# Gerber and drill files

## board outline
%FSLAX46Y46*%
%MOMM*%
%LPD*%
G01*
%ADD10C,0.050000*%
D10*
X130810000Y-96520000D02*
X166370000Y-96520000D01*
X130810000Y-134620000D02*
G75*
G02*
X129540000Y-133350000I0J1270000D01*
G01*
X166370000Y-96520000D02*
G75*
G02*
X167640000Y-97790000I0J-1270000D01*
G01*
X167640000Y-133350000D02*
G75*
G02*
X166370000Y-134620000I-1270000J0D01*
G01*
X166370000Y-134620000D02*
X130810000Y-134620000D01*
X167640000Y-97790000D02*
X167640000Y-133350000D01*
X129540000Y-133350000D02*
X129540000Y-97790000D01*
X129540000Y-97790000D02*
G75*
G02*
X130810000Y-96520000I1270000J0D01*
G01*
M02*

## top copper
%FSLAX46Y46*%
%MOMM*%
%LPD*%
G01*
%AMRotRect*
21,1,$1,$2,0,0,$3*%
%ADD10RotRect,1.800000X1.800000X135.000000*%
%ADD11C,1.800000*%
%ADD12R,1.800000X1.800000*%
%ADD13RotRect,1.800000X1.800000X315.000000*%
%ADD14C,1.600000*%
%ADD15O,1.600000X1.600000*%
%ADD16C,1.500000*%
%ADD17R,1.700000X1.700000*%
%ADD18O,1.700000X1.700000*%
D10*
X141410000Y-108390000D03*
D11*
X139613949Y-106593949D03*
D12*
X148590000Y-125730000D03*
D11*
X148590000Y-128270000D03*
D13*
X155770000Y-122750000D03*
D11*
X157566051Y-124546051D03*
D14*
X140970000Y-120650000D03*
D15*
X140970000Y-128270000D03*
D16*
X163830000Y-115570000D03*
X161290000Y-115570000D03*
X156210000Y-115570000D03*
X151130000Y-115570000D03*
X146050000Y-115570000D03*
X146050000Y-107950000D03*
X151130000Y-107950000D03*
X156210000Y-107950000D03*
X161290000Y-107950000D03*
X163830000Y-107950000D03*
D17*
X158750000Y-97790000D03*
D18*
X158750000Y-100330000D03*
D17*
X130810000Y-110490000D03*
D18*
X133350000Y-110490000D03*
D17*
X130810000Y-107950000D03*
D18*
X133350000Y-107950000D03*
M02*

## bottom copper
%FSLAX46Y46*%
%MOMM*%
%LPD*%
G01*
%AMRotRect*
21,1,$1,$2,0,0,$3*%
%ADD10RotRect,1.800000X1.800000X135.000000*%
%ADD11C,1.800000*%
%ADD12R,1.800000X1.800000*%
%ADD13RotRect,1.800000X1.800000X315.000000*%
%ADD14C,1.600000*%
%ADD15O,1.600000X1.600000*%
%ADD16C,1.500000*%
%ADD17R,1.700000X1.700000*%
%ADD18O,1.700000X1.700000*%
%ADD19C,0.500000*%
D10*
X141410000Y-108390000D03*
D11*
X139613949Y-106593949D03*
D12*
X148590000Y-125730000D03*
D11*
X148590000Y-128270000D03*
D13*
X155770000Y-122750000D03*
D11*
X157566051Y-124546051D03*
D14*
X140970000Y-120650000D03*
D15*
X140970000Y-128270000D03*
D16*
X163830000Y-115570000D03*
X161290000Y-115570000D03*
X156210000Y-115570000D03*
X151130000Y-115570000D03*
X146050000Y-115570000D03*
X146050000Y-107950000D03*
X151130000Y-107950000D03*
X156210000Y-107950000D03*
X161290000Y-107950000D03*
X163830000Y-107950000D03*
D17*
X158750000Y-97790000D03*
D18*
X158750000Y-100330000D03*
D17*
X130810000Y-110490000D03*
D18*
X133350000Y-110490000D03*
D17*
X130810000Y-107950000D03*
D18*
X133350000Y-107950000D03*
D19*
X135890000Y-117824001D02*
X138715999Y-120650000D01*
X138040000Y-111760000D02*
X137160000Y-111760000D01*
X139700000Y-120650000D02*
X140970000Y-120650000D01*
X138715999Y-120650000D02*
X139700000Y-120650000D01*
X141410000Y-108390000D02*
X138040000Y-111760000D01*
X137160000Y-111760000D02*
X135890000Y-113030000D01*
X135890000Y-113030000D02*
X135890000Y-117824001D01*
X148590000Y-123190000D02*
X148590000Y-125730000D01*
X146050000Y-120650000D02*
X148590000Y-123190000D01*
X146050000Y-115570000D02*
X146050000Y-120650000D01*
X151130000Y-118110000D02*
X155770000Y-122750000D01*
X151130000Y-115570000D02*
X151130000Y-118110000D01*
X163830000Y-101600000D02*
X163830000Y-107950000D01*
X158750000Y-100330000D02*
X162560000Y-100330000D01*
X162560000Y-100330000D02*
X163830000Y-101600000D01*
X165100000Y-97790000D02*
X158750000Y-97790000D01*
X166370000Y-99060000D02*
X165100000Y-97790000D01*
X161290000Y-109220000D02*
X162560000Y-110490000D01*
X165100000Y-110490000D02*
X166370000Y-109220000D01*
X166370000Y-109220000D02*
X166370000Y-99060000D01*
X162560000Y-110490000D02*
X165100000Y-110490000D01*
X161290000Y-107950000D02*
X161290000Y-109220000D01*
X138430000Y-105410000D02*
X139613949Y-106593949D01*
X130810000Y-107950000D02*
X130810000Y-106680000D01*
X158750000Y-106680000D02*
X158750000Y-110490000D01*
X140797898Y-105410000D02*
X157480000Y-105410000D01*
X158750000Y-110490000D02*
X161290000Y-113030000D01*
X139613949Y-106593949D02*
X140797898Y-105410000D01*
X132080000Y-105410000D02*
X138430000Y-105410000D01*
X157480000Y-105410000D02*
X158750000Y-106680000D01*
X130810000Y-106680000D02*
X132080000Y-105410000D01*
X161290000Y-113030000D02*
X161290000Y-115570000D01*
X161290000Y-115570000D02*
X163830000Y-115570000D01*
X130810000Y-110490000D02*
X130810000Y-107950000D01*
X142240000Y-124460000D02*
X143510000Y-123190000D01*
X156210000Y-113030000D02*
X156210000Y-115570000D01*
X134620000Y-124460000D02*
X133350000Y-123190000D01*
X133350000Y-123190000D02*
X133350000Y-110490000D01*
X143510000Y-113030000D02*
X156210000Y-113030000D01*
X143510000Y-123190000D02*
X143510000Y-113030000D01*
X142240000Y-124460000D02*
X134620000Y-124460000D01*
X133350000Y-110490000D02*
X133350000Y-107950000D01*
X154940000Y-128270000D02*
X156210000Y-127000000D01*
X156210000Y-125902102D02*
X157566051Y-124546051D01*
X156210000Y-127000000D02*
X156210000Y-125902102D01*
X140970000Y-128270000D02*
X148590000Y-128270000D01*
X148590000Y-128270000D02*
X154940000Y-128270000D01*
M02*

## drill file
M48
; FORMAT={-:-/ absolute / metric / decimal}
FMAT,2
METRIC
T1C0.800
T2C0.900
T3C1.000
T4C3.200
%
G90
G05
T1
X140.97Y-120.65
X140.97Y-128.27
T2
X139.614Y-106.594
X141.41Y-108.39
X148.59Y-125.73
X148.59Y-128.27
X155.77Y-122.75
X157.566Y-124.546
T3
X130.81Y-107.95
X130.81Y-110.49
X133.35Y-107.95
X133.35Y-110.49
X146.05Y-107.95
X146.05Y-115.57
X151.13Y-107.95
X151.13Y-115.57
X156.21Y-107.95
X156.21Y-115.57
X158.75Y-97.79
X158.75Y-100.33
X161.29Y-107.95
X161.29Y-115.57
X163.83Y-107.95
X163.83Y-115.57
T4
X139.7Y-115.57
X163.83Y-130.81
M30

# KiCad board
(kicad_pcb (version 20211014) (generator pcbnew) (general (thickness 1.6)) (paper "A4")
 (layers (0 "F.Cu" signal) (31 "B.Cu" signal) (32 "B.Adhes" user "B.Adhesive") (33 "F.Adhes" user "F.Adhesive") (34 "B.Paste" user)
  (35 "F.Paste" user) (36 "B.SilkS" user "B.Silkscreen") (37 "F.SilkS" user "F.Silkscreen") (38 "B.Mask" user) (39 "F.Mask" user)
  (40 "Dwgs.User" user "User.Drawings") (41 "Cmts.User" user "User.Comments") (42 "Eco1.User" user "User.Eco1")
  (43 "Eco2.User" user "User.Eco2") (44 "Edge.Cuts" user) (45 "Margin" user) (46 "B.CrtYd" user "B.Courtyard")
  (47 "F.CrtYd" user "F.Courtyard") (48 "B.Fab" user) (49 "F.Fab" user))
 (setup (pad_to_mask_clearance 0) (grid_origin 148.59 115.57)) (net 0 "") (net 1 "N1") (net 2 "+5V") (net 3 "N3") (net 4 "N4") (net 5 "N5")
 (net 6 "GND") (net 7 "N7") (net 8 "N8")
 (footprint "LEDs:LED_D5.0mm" (layer "F.Cu") (at 141.41 108.39 135)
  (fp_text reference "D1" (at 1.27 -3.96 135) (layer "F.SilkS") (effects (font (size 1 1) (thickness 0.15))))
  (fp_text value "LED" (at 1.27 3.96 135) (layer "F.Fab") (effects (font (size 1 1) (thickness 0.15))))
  (pad "1" thru_hole rect locked (at 0 0 135) (size 1.8 1.8) (drill 0.9) (layers *.Cu *.Mask) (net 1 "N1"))
  (pad "2" thru_hole circle locked (at 2.54 0 135) (size 1.8 1.8) (drill 0.9) (layers *.Cu *.Mask) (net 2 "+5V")))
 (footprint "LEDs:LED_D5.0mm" (layer "F.Cu") (at 148.59 125.73 -90)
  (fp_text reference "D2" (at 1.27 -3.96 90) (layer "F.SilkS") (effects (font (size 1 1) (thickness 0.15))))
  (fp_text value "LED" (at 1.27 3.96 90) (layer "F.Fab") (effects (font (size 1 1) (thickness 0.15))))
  (pad "1" thru_hole rect locked (at 0 0 270) (size 1.8 1.8) (drill 0.9) (layers *.Cu *.Mask) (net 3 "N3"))
  (pad "2" thru_hole circle locked (at 2.54 0 270) (size 1.8 1.8) (drill 0.9) (layers *.Cu *.Mask) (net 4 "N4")))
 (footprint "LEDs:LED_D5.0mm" (layer "F.Cu") (at 155.77 122.75 -45)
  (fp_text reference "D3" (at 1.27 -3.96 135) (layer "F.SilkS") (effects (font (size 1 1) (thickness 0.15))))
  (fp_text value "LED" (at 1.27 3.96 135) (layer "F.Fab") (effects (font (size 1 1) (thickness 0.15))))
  (pad "1" thru_hole rect locked (at 0 0 315) (size 1.8 1.8) (drill 0.9) (layers *.Cu *.Mask) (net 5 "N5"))
  (pad "2" thru_hole circle locked (at 2.54 0 315) (size 1.8 1.8) (drill 0.9) (layers *.Cu *.Mask) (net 4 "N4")))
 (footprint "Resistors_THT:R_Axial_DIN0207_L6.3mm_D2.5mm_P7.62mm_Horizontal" (layer "F.Cu") (at 140.97 120.65 -90)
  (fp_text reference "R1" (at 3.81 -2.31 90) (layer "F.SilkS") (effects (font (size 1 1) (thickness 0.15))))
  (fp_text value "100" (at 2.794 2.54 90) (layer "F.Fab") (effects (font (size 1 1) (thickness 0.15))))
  (pad "1" thru_hole circle locked (at 0 0 270) (size 1.6 1.6) (drill 0.8) (layers *.Cu *.Mask) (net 1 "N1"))
  (pad "2" thru_hole oval locked (at 7.62 0 270) (size 1.6 1.6) (drill 0.8) (layers *.Cu *.Mask) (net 4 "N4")))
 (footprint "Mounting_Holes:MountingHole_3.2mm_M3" (layer "F.Cu") (at 163.83 130.81 -90)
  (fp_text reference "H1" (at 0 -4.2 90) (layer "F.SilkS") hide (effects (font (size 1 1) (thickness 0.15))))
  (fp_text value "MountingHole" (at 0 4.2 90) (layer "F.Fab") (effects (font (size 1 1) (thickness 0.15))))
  (pad "" np_thru_hole circle locked (at 0 0 270) (size 3.2 3.2) (drill 3.2) (layers *.Cu *.Mask) (thermal_gap 2)))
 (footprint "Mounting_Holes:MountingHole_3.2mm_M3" (layer "F.Cu") (at 139.7 115.57 -90)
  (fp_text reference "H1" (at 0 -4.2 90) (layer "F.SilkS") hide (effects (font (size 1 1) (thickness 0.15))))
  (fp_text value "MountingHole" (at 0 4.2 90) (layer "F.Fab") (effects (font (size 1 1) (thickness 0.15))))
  (pad "" np_thru_hole circle locked (at 0 0 270) (size 3.2 3.2) (drill 3.2) (layers *.Cu *.Mask) (thermal_gap 2)))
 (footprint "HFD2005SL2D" (layer "B.Cu") (at 163.83 115.57 180)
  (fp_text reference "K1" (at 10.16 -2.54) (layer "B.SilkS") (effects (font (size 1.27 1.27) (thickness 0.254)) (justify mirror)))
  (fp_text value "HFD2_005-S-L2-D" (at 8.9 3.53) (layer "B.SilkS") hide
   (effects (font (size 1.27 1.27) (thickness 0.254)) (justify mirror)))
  (pad "1" thru_hole circle locked (at 0 0 90) (size 1.5 1.5) (drill 1) (layers *.Cu *.Mask "B.SilkS") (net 2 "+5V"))
  (pad "2" thru_hole circle locked (at 2.54 0 90) (size 1.5 1.5) (drill 1) (layers *.Cu *.Mask "B.SilkS") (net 2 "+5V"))
  (pad "4" thru_hole circle locked (at 7.62 0 90) (size 1.5 1.5) (drill 1) (layers *.Cu *.Mask "B.SilkS") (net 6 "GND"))
  (pad "6" thru_hole circle locked (at 12.7 0 90) (size 1.5 1.5) (drill 1) (layers *.Cu *.Mask "B.SilkS") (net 5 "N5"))
  (pad "8" thru_hole circle locked (at 17.78 0 90) (size 1.5 1.5) (drill 1) (layers *.Cu *.Mask "B.SilkS") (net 3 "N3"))
  (pad "9" thru_hole circle locked (at 17.78 7.62 90) (size 1.5 1.5) (drill 1) (layers *.Cu *.Mask "B.SilkS"))
  (pad "11" thru_hole circle locked (at 12.7 7.62 90) (size 1.5 1.5) (drill 1) (layers *.Cu *.Mask "B.SilkS"))
  (pad "13" thru_hole circle locked (at 7.62 7.62 90) (size 1.5 1.5) (drill 1) (layers *.Cu *.Mask "B.SilkS"))
  (pad "15" thru_hole circle locked (at 2.54 7.62 90) (size 1.5 1.5) (drill 1) (layers *.Cu *.Mask "B.SilkS") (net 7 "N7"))
  (pad "16" thru_hole circle locked (at 0 7.62 90) (size 1.5 1.5) (drill 1) (layers *.Cu *.Mask "B.SilkS") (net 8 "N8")))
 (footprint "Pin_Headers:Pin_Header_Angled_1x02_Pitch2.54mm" (layer "B.Cu") (at 158.75 97.79 180)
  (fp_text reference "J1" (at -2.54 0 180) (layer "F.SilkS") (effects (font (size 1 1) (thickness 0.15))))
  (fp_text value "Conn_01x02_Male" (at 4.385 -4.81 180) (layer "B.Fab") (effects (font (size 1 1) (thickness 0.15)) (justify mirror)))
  (pad "1" thru_hole rect locked (at 0 0 180) (size 1.7 1.7) (drill 1) (layers *.Cu *.Mask) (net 7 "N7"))
  (pad "2" thru_hole oval locked (at 0 -2.54 180) (size 1.7 1.7) (drill 1) (layers *.Cu *.Mask) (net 8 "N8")))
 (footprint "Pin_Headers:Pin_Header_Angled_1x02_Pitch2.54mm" (layer "B.Cu") (at 130.81 110.49 -90)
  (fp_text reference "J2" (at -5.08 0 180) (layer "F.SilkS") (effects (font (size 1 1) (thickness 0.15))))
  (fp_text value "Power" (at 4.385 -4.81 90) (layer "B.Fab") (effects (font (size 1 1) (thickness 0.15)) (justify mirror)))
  (pad "1" thru_hole rect locked (at 0 0 270) (size 1.7 1.7) (drill 1) (layers *.Cu *.Mask) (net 2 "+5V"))
  (pad "2" thru_hole oval locked (at 0 -2.54 270) (size 1.7 1.7) (drill 1) (layers *.Cu *.Mask) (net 6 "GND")))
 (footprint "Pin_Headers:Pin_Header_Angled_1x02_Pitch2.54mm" (layer "B.Cu") (at 130.81 107.95 -90)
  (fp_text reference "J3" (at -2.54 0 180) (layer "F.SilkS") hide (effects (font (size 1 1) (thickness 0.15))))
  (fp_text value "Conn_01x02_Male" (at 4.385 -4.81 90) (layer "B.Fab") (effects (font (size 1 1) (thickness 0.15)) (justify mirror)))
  (pad "1" thru_hole rect locked (at 0 0 270) (size 1.7 1.7) (drill 1) (layers *.Cu *.Mask) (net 2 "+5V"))
  (pad "2" thru_hole oval locked (at 0 -2.54 270) (size 1.7 1.7) (drill 1) (layers *.Cu *.Mask) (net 6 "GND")))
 (gr_line (start 130.81 96.52) (end 166.37 96.52) (layer "Edge.Cuts") (width 0.05))
 (gr_arc (start 130.81 134.62) (mid 129.911974 134.248026) (end 129.54 133.35) (layer "Edge.Cuts") (width 0.05))
 (gr_arc (start 166.37 96.52) (mid 167.268026 96.891974) (end 167.64 97.79) (layer "Edge.Cuts") (width 0.05))
 (gr_arc (start 167.64 133.35) (mid 167.268026 134.248026) (end 166.37 134.62) (layer "Edge.Cuts") (width 0.05))
 (gr_line (start 166.37 134.62) (end 130.81 134.62) (layer "Edge.Cuts") (width 0.05))
 (gr_line (start 167.64 97.79) (end 167.64 133.35) (layer "Edge.Cuts") (width 0.05))
 (gr_line (start 129.54 133.35) (end 129.54 97.79) (layer "Edge.Cuts") (width 0.05))
 (gr_arc (start 129.54 97.79) (mid 129.911974 96.891974) (end 130.81 96.52) (layer "Edge.Cuts") (width 0.05))
 (segment (start 135.89 117.824001) (end 138.715999 120.65) (width 0.5) (layer "B.Cu") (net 1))
 (segment (start 138.04 111.76) (end 137.16 111.76) (width 0.5) (layer "B.Cu") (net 1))
 (segment (start 139.7 120.65) (end 140.97 120.65) (width 0.5) (layer "B.Cu") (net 1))
 (segment (start 138.715999 120.65) (end 139.7 120.65) (width 0.5) (layer "B.Cu") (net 1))
 (segment (start 141.41 108.39) (end 138.04 111.76) (width 0.5) (layer "B.Cu") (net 1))
 (segment (start 137.16 111.76) (end 135.89 113.03) (width 0.5) (layer "B.Cu") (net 1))
 (segment (start 135.89 113.03) (end 135.89 117.824001) (width 0.5) (layer "B.Cu") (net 1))
 (segment (start 148.59 123.19) (end 148.59 125.73) (width 0.5) (layer "B.Cu") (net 3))
 (segment (start 146.05 120.65) (end 148.59 123.19) (width 0.5) (layer "B.Cu") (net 3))
 (segment (start 146.05 115.57) (end 146.05 120.65) (width 0.5) (layer "B.Cu") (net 3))
 (segment (start 151.13 118.11) (end 155.77 122.75) (width 0.5) (layer "B.Cu") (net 5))
 (segment (start 151.13 115.57) (end 151.13 118.11) (width 0.5) (layer "B.Cu") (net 5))
 (segment (start 163.83 101.6) (end 163.83 107.95) (width 0.5) (layer "B.Cu") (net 8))
 (segment (start 158.75 100.33) (end 162.56 100.33) (width 0.5) (layer "B.Cu") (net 8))
 (segment (start 162.56 100.33) (end 163.83 101.6) (width 0.5) (layer "B.Cu") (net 8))
 (segment (start 165.1 97.79) (end 158.75 97.79) (width 0.5) (layer "B.Cu") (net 7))
 (segment (start 166.37 99.06) (end 165.1 97.79) (width 0.5) (layer "B.Cu") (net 7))
 (segment (start 161.29 109.22) (end 162.56 110.49) (width 0.5) (layer "B.Cu") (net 7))
 (segment (start 165.1 110.49) (end 166.37 109.22) (width 0.5) (layer "B.Cu") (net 7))
 (segment (start 166.37 109.22) (end 166.37 99.06) (width 0.5) (layer "B.Cu") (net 7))
 (segment (start 162.56 110.49) (end 165.1 110.49) (width 0.5) (layer "B.Cu") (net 7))
 (segment (start 161.29 107.95) (end 161.29 109.22) (width 0.5) (layer "B.Cu") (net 7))
 (segment (start 138.43 105.41) (end 139.613949 106.593949) (width 0.5) (layer "B.Cu") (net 2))
 (segment (start 130.81 107.95) (end 130.81 106.68) (width 0.5) (layer "B.Cu") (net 2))
 (segment (start 158.75 106.68) (end 158.75 110.49) (width 0.5) (layer "B.Cu") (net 2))
 (segment (start 140.797898 105.41) (end 157.48 105.41) (width 0.5) (layer "B.Cu") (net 2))
 (segment (start 158.75 110.49) (end 161.29 113.03) (width 0.5) (layer "B.Cu") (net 2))
 (segment (start 139.613949 106.593949) (end 140.797898 105.41) (width 0.5) (layer "B.Cu") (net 2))
 (segment (start 132.08 105.41) (end 138.43 105.41) (width 0.5) (layer "B.Cu") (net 2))
 (segment (start 157.48 105.41) (end 158.75 106.68) (width 0.5) (layer "B.Cu") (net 2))
 (segment (start 130.81 106.68) (end 132.08 105.41) (width 0.5) (layer "B.Cu") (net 2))
 (segment (start 161.29 113.03) (end 161.29 115.57) (width 0.5) (layer "B.Cu") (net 2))
 (segment (start 161.29 115.57) (end 163.83 115.57) (width 0.5) (layer "B.Cu") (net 2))
 (segment (start 130.81 110.49) (end 130.81 107.95) (width 0.5) (layer "B.Cu") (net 2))
 (segment (start 142.24 124.46) (end 143.51 123.19) (width 0.5) (layer "B.Cu") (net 6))
 (segment (start 156.21 113.03) (end 156.21 115.57) (width 0.5) (layer "B.Cu") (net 6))
 (segment (start 134.62 124.46) (end 133.35 123.19) (width 0.5) (layer "B.Cu") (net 6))
 (segment (start 133.35 123.19) (end 133.35 110.49) (width 0.5) (layer "B.Cu") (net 6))
 (segment (start 143.51 113.03) (end 156.21 113.03) (width 0.5) (layer "B.Cu") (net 6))
 (segment (start 143.51 123.19) (end 143.51 113.03) (width 0.5) (layer "B.Cu") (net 6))
 (segment (start 142.24 124.46) (end 134.62 124.46) (width 0.5) (layer "B.Cu") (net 6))
 (segment (start 133.35 110.49) (end 133.35 107.95) (width 0.5) (layer "B.Cu") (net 6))
 (segment (start 154.94 128.27) (end 156.21 127) (width 0.5) (layer "B.Cu") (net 4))
 (segment (start 156.21 125.902102) (end 157.566051 124.546051) (width 0.5) (layer "B.Cu") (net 4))
 (segment (start 156.21 127) (end 156.21 125.902102) (width 0.5) (layer "B.Cu") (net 4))
 (segment (start 140.97 128.27) (end 148.59 128.27) (width 0.5) (layer "B.Cu") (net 4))
 (segment (start 148.59 128.27) (end 154.94 128.27) (width 0.5) (layer "B.Cu") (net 4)))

